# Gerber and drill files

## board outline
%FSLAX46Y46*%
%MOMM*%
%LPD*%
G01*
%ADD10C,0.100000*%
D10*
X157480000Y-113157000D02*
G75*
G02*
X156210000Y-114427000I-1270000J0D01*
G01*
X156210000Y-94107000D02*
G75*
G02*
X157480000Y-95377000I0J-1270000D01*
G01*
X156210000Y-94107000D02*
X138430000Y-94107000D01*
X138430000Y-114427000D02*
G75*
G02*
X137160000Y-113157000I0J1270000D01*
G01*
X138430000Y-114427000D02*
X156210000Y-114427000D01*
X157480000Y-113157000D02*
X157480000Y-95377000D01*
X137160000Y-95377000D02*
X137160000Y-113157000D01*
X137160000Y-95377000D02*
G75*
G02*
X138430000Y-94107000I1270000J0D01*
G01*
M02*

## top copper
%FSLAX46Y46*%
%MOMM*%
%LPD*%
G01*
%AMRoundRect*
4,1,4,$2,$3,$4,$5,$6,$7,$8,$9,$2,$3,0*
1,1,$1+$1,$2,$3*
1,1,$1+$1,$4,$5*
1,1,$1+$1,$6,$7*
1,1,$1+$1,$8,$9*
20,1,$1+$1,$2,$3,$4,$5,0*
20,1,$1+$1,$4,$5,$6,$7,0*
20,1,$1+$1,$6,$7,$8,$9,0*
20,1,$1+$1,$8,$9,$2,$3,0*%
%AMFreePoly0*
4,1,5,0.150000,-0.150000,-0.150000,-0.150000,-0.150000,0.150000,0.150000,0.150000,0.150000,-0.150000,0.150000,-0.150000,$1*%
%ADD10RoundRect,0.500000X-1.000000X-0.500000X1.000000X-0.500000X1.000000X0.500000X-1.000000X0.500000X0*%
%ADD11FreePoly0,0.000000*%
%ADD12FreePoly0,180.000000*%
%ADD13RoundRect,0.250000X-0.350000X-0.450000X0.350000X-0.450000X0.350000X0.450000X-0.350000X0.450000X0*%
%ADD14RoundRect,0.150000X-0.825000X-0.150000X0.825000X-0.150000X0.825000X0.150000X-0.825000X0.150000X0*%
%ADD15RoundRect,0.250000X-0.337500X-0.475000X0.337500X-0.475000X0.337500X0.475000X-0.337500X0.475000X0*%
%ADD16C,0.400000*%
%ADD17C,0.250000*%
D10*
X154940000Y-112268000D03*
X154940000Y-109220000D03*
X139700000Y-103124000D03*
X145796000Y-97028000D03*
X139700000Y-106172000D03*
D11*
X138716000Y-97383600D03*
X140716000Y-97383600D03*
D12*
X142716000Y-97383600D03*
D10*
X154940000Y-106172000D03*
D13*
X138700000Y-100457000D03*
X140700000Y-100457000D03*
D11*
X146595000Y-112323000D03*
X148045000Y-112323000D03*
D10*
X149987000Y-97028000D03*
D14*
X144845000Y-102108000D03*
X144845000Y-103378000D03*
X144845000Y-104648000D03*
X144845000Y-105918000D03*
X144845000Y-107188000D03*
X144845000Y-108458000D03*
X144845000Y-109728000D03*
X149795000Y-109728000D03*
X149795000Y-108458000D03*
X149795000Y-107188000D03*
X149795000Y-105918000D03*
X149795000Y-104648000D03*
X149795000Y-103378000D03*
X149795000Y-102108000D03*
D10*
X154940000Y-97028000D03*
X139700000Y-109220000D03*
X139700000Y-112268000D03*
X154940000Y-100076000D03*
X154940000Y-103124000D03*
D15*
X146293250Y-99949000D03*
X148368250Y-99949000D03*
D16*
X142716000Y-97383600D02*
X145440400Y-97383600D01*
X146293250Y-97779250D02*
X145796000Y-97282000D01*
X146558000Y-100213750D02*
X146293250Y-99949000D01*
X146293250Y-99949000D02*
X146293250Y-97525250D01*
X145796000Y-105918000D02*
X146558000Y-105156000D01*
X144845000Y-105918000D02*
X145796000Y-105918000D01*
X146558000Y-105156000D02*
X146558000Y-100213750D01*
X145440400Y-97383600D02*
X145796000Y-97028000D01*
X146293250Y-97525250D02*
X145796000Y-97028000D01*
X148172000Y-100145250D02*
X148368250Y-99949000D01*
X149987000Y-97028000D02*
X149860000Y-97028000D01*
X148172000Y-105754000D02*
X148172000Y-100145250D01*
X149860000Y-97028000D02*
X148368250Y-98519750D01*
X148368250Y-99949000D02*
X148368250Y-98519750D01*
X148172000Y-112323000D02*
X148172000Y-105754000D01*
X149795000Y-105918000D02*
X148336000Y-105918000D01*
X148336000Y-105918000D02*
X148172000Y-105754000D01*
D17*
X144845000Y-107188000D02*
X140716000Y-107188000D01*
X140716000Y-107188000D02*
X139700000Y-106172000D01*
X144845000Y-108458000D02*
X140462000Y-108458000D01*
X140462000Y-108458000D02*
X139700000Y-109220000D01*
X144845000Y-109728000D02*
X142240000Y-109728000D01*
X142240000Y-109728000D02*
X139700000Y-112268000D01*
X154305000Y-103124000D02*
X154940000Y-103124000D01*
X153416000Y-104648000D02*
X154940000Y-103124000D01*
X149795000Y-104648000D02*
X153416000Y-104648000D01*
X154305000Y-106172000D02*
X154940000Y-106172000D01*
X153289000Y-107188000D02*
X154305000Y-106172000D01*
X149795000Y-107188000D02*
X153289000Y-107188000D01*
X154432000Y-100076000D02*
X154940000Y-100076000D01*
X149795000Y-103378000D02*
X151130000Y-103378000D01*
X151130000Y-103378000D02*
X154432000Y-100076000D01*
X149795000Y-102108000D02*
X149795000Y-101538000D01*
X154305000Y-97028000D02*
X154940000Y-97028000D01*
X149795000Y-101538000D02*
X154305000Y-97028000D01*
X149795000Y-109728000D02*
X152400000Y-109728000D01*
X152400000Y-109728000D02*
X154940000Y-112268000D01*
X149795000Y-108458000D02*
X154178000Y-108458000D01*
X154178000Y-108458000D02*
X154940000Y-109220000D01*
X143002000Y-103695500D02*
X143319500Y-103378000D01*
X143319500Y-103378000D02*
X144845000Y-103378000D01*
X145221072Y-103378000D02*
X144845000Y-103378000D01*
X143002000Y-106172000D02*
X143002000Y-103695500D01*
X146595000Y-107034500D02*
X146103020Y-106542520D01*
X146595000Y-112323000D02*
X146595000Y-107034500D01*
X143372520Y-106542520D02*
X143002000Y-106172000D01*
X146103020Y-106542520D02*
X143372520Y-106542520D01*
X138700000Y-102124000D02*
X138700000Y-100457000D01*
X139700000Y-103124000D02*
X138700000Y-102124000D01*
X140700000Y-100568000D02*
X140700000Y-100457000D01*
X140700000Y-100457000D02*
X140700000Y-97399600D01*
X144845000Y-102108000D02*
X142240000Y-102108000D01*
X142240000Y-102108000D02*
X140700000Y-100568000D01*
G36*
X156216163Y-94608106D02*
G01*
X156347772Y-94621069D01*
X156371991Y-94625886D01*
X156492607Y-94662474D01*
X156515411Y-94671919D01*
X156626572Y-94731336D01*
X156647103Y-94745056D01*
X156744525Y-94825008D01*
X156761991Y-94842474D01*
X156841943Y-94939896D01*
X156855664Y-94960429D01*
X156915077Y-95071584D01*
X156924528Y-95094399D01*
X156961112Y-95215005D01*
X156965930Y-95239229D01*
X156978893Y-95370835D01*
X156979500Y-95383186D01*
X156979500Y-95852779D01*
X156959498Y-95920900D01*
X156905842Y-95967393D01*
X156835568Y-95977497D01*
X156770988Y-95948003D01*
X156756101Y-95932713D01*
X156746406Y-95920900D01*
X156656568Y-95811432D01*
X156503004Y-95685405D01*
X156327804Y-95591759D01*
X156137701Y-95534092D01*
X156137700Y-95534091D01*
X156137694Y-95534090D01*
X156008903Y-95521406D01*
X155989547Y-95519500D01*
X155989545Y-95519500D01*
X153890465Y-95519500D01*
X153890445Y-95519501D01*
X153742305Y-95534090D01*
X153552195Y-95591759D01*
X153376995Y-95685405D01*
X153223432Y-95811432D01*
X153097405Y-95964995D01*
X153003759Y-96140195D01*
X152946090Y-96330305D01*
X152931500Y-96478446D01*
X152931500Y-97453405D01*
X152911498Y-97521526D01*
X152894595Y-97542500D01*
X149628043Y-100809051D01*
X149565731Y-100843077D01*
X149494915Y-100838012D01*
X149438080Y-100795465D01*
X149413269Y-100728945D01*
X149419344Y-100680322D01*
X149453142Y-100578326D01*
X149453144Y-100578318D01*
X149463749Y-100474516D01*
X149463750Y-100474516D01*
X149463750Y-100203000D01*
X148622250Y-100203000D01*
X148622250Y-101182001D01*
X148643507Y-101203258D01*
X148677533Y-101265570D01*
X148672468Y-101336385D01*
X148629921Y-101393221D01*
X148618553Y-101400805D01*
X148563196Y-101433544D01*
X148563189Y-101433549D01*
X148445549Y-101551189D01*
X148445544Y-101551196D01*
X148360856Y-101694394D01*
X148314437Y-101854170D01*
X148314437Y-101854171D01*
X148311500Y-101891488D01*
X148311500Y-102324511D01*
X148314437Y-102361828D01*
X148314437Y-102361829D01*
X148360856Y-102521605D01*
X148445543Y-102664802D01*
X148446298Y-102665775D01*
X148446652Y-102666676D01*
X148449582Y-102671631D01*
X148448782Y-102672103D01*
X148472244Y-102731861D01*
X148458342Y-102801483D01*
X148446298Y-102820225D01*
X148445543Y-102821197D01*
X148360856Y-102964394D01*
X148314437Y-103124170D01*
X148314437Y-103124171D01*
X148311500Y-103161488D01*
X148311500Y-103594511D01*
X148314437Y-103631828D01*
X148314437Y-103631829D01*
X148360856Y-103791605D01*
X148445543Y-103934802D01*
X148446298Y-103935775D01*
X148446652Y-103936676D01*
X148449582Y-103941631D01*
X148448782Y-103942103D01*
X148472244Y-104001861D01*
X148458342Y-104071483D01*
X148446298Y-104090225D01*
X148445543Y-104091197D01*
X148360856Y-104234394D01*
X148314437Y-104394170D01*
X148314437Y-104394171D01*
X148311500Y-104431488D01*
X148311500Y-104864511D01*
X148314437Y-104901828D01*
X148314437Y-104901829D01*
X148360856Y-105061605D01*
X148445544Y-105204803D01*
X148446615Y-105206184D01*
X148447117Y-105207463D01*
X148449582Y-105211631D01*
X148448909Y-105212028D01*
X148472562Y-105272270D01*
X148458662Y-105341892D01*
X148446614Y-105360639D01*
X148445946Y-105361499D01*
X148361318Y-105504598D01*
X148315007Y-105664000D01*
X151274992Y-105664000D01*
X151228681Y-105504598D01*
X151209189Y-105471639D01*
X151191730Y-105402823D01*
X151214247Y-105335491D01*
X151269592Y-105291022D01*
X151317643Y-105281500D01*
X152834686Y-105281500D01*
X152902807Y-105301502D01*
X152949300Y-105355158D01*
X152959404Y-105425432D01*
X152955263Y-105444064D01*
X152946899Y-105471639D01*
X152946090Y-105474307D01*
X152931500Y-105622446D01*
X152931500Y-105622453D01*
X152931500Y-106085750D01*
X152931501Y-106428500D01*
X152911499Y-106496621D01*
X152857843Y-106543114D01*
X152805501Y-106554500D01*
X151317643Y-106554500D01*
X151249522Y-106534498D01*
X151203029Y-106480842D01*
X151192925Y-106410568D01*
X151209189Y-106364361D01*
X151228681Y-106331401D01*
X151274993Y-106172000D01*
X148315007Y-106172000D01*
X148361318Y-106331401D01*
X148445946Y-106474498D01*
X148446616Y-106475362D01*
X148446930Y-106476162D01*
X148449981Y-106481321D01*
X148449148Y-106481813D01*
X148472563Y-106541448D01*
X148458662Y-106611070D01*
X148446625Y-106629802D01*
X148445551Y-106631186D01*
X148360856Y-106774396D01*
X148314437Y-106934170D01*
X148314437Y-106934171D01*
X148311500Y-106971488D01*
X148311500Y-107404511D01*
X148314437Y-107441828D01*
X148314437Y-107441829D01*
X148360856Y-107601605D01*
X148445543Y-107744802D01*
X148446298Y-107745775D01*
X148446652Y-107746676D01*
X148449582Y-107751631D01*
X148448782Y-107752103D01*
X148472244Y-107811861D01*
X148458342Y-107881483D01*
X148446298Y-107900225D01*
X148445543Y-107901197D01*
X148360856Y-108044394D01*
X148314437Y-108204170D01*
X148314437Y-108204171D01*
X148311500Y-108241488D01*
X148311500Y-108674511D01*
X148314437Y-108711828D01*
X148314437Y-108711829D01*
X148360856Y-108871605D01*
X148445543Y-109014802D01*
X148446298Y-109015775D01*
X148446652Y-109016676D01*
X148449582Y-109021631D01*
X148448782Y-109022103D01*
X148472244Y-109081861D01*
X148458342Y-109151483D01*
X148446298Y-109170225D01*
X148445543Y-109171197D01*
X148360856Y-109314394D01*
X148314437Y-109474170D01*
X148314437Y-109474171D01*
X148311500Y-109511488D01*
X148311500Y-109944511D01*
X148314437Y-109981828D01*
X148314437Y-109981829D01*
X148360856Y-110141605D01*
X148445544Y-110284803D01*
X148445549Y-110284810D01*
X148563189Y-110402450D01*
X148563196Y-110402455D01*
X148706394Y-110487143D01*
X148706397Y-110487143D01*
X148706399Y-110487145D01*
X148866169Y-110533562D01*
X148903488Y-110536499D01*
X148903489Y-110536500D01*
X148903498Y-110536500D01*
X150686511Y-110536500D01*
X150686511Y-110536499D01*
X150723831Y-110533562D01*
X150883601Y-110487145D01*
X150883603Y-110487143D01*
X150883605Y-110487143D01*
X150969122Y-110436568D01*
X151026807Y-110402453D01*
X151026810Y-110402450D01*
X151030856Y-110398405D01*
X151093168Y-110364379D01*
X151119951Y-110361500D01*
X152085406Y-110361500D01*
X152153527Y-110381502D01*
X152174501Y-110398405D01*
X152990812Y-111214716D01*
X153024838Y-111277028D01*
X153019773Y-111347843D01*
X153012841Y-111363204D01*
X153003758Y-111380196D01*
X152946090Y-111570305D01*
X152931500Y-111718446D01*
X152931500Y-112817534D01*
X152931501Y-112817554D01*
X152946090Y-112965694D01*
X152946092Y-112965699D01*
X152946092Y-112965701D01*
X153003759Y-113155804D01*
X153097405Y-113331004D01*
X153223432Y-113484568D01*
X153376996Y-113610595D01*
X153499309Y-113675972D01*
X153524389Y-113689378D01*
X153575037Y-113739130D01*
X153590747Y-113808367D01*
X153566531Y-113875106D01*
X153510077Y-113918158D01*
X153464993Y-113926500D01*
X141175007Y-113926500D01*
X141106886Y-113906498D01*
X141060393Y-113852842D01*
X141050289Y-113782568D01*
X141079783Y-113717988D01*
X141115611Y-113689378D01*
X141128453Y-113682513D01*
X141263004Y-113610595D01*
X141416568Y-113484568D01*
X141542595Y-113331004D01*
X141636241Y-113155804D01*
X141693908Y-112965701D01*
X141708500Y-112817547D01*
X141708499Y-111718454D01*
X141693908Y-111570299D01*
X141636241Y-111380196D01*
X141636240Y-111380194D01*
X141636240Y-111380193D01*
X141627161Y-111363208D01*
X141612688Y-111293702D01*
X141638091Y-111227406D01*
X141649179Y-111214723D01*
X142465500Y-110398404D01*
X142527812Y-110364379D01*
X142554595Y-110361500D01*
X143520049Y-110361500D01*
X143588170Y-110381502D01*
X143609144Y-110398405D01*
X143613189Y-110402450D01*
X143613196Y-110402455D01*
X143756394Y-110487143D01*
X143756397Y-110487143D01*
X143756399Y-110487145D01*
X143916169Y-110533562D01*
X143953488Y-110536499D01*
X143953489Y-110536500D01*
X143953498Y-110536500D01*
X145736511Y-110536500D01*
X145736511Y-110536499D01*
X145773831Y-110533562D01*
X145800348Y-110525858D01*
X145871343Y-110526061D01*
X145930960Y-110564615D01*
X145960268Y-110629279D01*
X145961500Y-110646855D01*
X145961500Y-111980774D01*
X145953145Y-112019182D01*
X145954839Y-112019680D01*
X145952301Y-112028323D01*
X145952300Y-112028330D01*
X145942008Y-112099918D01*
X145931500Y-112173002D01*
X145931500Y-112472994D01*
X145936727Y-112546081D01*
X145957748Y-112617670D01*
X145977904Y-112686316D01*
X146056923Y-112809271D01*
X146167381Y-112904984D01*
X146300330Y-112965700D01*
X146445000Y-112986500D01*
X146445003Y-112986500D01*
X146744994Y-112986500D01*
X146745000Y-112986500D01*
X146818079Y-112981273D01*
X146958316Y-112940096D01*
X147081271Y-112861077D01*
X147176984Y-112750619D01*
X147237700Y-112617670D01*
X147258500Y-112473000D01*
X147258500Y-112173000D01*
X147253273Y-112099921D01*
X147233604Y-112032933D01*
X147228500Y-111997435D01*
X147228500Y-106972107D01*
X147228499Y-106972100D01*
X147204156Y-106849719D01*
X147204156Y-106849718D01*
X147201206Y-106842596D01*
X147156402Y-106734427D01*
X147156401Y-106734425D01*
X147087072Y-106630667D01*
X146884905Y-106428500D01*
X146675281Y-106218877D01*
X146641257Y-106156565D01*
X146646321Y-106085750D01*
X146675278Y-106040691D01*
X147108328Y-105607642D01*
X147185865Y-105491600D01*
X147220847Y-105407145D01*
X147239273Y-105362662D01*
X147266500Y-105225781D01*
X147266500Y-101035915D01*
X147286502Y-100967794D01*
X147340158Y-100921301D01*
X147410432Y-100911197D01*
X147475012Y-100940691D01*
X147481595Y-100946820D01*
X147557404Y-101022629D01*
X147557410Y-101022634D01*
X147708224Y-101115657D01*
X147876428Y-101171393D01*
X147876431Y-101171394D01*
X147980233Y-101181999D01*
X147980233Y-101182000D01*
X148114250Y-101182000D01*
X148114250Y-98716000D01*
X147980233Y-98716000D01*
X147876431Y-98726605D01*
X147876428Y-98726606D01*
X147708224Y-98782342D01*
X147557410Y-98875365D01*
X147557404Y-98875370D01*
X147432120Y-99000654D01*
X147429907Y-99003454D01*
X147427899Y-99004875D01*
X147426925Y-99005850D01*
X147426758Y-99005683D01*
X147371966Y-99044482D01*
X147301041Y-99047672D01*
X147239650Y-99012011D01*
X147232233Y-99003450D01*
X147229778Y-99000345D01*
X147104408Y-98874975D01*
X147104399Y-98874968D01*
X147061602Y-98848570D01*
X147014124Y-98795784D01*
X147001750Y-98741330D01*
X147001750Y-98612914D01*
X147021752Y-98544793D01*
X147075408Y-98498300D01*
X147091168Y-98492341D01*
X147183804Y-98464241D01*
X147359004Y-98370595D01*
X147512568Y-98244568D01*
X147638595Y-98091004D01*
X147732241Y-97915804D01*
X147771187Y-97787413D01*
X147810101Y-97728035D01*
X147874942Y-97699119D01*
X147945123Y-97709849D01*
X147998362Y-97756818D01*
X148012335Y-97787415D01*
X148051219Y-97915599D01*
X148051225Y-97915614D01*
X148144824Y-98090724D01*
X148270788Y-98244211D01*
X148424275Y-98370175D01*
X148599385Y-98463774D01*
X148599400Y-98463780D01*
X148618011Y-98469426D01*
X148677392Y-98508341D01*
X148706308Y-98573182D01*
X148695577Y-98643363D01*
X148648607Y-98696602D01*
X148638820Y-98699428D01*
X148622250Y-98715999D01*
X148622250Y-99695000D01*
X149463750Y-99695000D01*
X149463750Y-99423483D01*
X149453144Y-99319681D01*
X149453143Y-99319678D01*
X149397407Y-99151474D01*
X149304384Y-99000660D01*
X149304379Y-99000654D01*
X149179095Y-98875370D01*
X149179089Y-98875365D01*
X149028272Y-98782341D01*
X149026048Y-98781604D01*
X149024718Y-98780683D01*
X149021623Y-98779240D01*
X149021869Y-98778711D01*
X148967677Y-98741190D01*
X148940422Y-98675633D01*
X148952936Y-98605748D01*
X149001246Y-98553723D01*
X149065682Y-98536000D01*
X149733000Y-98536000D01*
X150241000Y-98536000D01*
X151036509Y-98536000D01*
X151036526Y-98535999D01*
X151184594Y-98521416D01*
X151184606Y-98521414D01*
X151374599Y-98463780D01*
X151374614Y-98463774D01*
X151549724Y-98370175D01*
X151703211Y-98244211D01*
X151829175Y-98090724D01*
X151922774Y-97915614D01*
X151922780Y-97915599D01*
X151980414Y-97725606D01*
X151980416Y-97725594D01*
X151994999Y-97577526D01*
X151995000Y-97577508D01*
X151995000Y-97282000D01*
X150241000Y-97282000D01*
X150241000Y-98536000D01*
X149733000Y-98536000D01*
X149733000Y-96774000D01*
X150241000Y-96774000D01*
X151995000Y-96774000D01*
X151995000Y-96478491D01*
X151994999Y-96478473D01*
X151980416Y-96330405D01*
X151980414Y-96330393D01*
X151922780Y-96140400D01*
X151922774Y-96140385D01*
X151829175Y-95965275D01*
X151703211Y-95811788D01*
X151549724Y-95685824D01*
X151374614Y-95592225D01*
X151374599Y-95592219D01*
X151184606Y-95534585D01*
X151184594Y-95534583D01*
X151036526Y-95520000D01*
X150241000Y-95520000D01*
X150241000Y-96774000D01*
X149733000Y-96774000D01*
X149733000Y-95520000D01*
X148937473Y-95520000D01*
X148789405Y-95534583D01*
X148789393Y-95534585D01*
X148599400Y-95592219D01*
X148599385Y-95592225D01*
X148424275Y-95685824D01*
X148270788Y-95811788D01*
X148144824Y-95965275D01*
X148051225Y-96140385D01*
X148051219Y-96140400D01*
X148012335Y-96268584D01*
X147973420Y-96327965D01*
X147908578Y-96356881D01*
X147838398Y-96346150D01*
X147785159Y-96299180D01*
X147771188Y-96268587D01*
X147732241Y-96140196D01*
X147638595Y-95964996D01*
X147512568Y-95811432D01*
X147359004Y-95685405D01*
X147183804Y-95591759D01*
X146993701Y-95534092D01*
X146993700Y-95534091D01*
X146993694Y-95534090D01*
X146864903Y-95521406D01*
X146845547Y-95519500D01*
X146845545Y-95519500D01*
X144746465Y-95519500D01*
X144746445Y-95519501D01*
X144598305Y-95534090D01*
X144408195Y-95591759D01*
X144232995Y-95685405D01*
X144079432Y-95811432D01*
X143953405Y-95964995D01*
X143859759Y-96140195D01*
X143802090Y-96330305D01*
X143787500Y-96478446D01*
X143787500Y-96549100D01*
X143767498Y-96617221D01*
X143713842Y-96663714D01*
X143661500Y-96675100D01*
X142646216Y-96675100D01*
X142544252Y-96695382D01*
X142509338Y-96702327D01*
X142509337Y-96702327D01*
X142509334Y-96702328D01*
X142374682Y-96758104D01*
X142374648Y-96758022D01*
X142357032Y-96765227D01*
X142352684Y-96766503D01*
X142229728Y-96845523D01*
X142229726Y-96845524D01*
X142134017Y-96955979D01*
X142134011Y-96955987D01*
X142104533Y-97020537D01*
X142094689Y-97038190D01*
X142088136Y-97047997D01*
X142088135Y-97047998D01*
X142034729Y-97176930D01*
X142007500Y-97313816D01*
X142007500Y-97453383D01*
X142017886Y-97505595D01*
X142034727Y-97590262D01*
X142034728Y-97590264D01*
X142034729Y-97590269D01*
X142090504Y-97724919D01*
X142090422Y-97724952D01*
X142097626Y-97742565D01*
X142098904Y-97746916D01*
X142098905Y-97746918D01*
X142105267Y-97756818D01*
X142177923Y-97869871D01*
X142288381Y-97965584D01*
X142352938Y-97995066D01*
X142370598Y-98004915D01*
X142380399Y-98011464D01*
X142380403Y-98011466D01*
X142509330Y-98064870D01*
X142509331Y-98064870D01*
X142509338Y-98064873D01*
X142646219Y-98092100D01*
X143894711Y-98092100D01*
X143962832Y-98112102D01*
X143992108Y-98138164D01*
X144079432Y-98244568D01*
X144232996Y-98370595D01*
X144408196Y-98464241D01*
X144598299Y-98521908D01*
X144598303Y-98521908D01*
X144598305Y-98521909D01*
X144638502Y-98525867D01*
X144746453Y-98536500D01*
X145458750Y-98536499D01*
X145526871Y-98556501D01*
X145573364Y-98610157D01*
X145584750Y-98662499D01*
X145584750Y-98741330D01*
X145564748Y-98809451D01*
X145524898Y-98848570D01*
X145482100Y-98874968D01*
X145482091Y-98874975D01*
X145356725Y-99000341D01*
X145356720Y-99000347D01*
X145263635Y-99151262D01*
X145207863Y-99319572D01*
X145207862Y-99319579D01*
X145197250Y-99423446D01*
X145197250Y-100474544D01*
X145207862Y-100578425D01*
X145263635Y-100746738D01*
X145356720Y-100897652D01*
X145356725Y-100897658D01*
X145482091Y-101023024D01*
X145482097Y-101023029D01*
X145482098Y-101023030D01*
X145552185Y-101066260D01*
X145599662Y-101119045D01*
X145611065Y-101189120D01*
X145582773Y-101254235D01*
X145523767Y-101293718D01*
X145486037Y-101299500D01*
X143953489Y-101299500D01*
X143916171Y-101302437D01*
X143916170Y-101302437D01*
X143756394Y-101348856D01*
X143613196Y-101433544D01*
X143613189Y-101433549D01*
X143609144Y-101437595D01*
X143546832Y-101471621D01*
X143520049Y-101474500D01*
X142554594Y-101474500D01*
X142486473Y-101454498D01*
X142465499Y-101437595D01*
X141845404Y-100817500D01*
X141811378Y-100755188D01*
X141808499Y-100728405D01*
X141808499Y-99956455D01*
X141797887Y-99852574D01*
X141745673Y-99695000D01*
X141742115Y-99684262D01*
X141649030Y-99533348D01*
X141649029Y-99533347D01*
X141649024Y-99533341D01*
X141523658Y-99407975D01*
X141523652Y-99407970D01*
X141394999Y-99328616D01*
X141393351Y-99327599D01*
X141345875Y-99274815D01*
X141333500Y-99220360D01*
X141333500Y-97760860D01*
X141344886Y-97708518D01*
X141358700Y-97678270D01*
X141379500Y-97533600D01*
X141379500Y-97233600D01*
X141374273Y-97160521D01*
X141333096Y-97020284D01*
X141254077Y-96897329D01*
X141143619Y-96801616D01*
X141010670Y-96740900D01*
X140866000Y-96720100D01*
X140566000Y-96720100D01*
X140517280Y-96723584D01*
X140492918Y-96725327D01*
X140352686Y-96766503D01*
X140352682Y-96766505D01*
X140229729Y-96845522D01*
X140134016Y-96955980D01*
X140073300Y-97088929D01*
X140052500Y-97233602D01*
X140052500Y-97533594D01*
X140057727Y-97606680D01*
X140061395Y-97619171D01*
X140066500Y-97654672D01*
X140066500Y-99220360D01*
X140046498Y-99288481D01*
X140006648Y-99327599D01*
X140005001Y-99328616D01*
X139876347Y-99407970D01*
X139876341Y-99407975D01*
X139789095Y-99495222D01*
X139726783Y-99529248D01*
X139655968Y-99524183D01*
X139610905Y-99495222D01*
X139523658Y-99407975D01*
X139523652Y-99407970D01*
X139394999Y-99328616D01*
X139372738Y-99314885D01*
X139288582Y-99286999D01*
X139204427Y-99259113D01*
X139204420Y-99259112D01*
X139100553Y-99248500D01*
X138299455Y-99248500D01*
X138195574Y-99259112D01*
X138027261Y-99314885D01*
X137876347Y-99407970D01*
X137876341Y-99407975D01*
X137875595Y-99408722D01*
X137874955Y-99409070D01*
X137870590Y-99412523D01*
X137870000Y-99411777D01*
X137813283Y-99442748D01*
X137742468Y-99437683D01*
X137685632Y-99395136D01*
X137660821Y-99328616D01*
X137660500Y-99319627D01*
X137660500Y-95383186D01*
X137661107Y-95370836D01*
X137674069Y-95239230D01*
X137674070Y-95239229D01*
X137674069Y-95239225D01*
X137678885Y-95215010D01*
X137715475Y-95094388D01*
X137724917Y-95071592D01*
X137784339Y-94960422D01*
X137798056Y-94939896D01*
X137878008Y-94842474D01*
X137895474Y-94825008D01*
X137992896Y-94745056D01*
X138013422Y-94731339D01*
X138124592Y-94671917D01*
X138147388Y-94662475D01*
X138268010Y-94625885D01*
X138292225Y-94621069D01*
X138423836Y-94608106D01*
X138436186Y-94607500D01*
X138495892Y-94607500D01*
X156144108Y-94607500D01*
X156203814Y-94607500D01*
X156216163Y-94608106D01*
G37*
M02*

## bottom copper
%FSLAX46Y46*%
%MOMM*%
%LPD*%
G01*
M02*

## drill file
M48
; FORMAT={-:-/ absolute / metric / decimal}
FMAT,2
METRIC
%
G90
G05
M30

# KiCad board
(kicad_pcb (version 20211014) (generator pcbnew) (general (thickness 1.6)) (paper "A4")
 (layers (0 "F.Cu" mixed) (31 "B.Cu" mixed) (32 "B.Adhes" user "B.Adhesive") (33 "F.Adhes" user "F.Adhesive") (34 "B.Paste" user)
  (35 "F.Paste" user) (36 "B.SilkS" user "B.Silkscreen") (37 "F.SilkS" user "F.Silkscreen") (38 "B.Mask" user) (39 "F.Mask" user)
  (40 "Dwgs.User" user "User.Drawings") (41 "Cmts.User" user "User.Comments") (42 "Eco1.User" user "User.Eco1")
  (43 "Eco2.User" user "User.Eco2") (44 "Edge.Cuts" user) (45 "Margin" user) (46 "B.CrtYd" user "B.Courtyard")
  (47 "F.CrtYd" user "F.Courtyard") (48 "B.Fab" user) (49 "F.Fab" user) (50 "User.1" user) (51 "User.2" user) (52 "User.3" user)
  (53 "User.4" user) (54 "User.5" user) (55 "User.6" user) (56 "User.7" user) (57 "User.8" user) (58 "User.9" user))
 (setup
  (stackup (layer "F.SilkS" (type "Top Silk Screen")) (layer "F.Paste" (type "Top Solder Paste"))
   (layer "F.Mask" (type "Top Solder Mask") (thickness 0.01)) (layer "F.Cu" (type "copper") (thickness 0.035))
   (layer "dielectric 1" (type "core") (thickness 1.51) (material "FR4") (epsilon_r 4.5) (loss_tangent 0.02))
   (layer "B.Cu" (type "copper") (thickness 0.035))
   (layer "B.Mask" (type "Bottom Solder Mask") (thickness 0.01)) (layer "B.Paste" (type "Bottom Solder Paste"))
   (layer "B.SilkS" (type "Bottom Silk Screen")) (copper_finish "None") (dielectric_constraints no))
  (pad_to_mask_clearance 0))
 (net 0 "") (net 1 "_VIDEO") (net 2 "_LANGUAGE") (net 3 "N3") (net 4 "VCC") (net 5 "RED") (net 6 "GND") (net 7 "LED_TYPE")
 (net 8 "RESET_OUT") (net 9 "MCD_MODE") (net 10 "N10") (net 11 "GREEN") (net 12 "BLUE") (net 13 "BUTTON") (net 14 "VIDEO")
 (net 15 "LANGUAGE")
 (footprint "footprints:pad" (layer "F.Cu") (at 154.94 112.268)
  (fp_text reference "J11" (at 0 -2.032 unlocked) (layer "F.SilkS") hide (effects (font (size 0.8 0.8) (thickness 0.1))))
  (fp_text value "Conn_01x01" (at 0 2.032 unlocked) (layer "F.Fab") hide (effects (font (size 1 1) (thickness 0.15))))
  (pad "1" smd roundrect (at 0 0) (size 3 2) (layers "F.Cu" "F.Paste" "F.Mask") (roundrect_rratio 0.25) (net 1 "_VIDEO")))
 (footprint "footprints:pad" (layer "F.Cu") (at 154.94 109.22)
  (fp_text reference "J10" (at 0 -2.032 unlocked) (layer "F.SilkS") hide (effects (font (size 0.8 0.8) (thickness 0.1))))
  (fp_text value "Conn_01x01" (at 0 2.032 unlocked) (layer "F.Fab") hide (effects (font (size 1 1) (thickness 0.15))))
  (pad "1" smd roundrect (at 0 0) (size 3 2) (layers "F.Cu" "F.Paste" "F.Mask") (roundrect_rratio 0.25) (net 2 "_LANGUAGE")))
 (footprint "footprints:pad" (layer "F.Cu") (at 139.7 103.124)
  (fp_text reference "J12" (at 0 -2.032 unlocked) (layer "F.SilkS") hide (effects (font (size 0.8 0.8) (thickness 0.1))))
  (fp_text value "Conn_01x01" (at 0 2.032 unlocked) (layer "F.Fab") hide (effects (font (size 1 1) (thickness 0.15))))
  (pad "1" smd roundrect (at 0 0) (size 3 2) (layers "F.Cu" "F.Paste" "F.Mask") (roundrect_rratio 0.25) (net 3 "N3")))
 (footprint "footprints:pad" (layer "F.Cu") (at 145.796 97.028)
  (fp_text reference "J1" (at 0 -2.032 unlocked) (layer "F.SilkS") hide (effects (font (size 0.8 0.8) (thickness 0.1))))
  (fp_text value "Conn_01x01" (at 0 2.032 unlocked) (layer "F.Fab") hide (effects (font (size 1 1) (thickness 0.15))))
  (pad "1" smd roundrect (at 0 0) (size 3 2) (layers "F.Cu" "F.Paste" "F.Mask") (roundrect_rratio 0.25) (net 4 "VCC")))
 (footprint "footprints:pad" (layer "F.Cu") (at 139.7 106.172)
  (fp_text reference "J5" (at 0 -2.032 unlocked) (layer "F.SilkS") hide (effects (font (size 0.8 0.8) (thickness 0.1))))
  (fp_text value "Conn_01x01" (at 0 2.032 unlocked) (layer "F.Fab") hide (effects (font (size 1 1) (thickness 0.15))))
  (pad "1" smd roundrect (at 0 0) (size 3 2) (layers "F.Cu" "F.Paste" "F.Mask") (roundrect_rratio 0.25) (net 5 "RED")))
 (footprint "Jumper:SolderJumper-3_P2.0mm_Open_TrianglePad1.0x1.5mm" (layer "F.Cu") (at 140.716 97.3836)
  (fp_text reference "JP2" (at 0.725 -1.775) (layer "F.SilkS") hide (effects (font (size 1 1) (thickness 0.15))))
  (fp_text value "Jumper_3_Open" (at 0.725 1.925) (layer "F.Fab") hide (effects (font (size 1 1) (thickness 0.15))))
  (pad "" smd rect (at -1.2 0) (size 1.5 1.5) (layers "F.Mask"))
  (pad "" smd rect (at 1.2 0) (size 1.5 1.5) (layers "F.Mask"))
  (pad "1" smd custom (at -2 0) (size 0.3 0.3) (layers "F.Cu" "F.Mask") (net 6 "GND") (zone_connect 2)
   (options (clearance outline) (anchor rect)) (primitives))
  (pad "2" smd custom (at 0 0) (size 0.3 0.3) (layers "F.Cu") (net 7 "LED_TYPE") (zone_connect 2)
   (options (clearance outline) (anchor rect)) (primitives))
  (pad "3" smd custom (at 2 0 180) (size 0.3 0.3) (layers "F.Cu" "F.Mask") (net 4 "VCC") (zone_connect 2)
   (options (clearance outline) (anchor rect)) (primitives)))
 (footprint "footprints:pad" (layer "F.Cu") (at 154.94 106.172)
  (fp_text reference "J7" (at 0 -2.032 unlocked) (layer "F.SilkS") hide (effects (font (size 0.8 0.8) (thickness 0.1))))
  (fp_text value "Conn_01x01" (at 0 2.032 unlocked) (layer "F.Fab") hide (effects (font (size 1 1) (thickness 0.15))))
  (pad "1" smd roundrect (at 0 0) (size 3 2) (layers "F.Cu" "F.Paste" "F.Mask") (roundrect_rratio 0.25) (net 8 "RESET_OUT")))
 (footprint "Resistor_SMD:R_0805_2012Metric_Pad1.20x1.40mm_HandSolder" (layer "F.Cu") (at 139.7 100.457)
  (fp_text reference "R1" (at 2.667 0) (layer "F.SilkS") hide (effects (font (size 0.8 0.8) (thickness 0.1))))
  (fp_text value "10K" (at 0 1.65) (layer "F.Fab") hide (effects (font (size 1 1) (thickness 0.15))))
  (pad "1" smd roundrect (at -1 0) (size 1.2 1.4) (layers "F.Cu" "F.Paste" "F.Mask") (roundrect_rratio 0.2083333333) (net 3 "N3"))
  (pad "2" smd roundrect (at 1 0) (size 1.2 1.4) (layers "F.Cu" "F.Paste" "F.Mask") (roundrect_rratio 0.2083333333) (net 7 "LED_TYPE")))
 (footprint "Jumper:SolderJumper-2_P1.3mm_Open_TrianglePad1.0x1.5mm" (layer "F.Cu") (at 147.32 112.323)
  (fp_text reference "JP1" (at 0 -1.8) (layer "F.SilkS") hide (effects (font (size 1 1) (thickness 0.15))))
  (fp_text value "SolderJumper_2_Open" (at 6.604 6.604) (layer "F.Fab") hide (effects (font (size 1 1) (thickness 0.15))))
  (pad "1" smd custom (at -0.725 0) (size 0.3 0.3) (layers "F.Cu" "F.Mask") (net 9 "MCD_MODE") (zone_connect 2)
   (options (clearance outline) (anchor rect)) (primitives))
  (pad "2" smd custom (at 0.725 0) (size 0.3 0.3) (layers "F.Cu" "F.Mask") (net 6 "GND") (zone_connect 2)
   (options (clearance outline) (anchor rect)) (primitives)))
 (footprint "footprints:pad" (layer "F.Cu") (at 149.987 97.028)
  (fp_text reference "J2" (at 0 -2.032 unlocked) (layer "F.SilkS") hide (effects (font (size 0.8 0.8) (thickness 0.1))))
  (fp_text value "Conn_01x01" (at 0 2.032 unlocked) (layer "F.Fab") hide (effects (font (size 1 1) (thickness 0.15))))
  (pad "1" smd roundrect (at 0 0) (size 3 2) (layers "F.Cu" "F.Paste" "F.Mask") (roundrect_rratio 0.25) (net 6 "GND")))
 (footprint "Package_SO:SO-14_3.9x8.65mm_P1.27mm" (layer "F.Cu") (at 147.32 105.918)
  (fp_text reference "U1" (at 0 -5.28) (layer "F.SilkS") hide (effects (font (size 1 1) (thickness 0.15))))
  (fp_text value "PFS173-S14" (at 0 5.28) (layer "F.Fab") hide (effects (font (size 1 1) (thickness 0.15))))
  (pad "1" smd roundrect (at -2.475 -3.81) (size 1.95 0.6) (layers "F.Cu" "F.Paste" "F.Mask") (roundrect_rratio 0.25) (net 7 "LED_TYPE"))
  (pad "2" smd roundrect (at -2.475 -2.54) (size 1.95 0.6) (layers "F.Cu" "F.Paste" "F.Mask") (roundrect_rratio 0.25) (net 9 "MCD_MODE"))
  (pad "3" smd roundrect (at -2.475 -1.27) (size 1.95 0.6) (layers "F.Cu" "F.Paste" "F.Mask") (roundrect_rratio 0.25) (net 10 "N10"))
  (pad "4" smd roundrect (at -2.475 0) (size 1.95 0.6) (layers "F.Cu" "F.Paste" "F.Mask") (roundrect_rratio 0.25) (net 4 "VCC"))
  (pad "5" smd roundrect (at -2.475 1.27) (size 1.95 0.6) (layers "F.Cu" "F.Paste" "F.Mask") (roundrect_rratio 0.25) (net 5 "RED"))
  (pad "6" smd roundrect (at -2.475 2.54) (size 1.95 0.6) (layers "F.Cu" "F.Paste" "F.Mask") (roundrect_rratio 0.25) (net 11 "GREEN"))
  (pad "7" smd roundrect (at -2.475 3.81) (size 1.95 0.6) (layers "F.Cu" "F.Paste" "F.Mask") (roundrect_rratio 0.25) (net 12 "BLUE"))
  (pad "8" smd roundrect (at 2.475 3.81) (size 1.95 0.6) (layers "F.Cu" "F.Paste" "F.Mask") (roundrect_rratio 0.25) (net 1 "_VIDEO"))
  (pad "9" smd roundrect (at 2.475 2.54) (size 1.95 0.6) (layers "F.Cu" "F.Paste" "F.Mask") (roundrect_rratio 0.25) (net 2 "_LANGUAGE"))
  (pad "10" smd roundrect (at 2.475 1.27) (size 1.95 0.6) (layers "F.Cu" "F.Paste" "F.Mask") (roundrect_rratio 0.25) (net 8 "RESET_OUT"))
  (pad "11" smd roundrect (at 2.475 0) (size 1.95 0.6) (layers "F.Cu" "F.Paste" "F.Mask") (roundrect_rratio 0.25) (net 6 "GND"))
  (pad "12" smd roundrect (at 2.475 -1.27) (size 1.95 0.6) (layers "F.Cu" "F.Paste" "F.Mask") (roundrect_rratio 0.25) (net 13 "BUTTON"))
  (pad "13" smd roundrect (at 2.475 -2.54) (size 1.95 0.6) (layers "F.Cu" "F.Paste" "F.Mask") (roundrect_rratio 0.25) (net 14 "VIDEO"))
  (pad "14" smd roundrect (at 2.475 -3.81) (size 1.95 0.6) (layers "F.Cu" "F.Paste" "F.Mask") (roundrect_rratio 0.25) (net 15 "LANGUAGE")))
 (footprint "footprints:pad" (layer "F.Cu") (at 154.94 97.028)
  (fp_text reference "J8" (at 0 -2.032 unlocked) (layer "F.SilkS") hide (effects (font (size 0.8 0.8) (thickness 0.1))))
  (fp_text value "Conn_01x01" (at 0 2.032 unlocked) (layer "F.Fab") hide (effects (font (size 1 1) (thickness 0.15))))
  (pad "1" smd roundrect (at 0 0) (size 3 2) (layers "F.Cu" "F.Paste" "F.Mask") (roundrect_rratio 0.25) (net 15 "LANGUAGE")))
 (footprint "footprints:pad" (layer "F.Cu") (at 139.7 109.22)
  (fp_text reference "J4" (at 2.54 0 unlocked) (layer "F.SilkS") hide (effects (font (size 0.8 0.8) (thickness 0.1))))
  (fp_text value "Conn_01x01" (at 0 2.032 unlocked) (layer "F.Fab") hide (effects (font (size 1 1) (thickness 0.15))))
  (pad "1" smd roundrect (at 0 0) (size 3 2) (layers "F.Cu" "F.Paste" "F.Mask") (roundrect_rratio 0.25) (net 11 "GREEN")))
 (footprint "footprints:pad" (layer "F.Cu") (at 139.7 112.268)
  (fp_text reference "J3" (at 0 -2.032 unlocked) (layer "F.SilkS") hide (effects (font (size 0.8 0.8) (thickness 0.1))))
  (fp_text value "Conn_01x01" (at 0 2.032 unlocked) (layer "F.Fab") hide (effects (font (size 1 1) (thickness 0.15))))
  (pad "1" smd roundrect (at 0 0) (size 3 2) (layers "F.Cu" "F.Paste" "F.Mask") (roundrect_rratio 0.25) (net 12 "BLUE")))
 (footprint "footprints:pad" (layer "F.Cu") (at 154.94 100.076)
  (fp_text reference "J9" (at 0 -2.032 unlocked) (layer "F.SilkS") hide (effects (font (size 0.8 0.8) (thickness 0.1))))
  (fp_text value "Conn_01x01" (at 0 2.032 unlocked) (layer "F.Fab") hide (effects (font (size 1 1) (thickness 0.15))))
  (pad "1" smd roundrect (at 0 0) (size 3 2) (layers "F.Cu" "F.Paste" "F.Mask") (roundrect_rratio 0.25) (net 14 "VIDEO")))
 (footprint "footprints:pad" (layer "F.Cu") (at 154.94 103.124)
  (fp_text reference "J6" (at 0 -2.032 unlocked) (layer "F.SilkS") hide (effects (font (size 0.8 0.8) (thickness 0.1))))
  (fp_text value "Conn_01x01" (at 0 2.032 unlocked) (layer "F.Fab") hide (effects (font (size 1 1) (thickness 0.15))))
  (pad "1" smd roundrect (at 0 0) (size 3 2) (layers "F.Cu" "F.Paste" "F.Mask") (roundrect_rratio 0.25) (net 13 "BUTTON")))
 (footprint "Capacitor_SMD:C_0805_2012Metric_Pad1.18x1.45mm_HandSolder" (layer "F.Cu") (at 147.33075 99.949)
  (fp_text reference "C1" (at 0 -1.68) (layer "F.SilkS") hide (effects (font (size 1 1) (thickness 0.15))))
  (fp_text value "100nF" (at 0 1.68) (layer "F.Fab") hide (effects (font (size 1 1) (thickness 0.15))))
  (pad "1" smd roundrect (at -1.0375 0) (size 1.175 1.45) (layers "F.Cu" "F.Paste" "F.Mask") (roundrect_rratio 0.2127659574) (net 4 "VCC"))
  (pad "2" smd roundrect (at 1.0375 0) (size 1.175 1.45) (layers "F.Cu" "F.Paste" "F.Mask") (roundrect_rratio 0.2127659574) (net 6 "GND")))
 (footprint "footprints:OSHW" (layer "B.Cu") (at 144.399 98.298 180)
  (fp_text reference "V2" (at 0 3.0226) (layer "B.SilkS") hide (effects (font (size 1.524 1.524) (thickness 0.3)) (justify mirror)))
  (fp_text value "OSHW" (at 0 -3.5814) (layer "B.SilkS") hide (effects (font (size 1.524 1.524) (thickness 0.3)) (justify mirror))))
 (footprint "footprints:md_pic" (layer "B.Cu") (at 151.257 98.171 180)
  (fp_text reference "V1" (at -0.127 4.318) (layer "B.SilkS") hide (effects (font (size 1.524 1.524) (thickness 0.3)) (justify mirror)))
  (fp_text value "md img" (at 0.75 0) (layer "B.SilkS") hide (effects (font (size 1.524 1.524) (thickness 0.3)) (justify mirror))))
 (gr_arc (start 157.48 113.157) (mid 157.108026 114.055026) (end 156.21 114.427) (layer "Edge.Cuts") (width 0.1))
 (gr_arc (start 156.21 94.107) (mid 157.108026 94.478974) (end 157.48 95.377) (layer "Edge.Cuts") (width 0.1))
 (gr_line (start 156.21 94.107) (end 138.43 94.107) (layer "Edge.Cuts") (width 0.1))
 (gr_arc (start 138.43 114.427) (mid 137.531974 114.055026) (end 137.16 113.157) (layer "Edge.Cuts") (width 0.1))
 (gr_line (start 138.43 114.427) (end 156.21 114.427) (layer "Edge.Cuts") (width 0.1))
 (gr_line (start 157.48 113.157) (end 157.48 95.377) (layer "Edge.Cuts") (width 0.1))
 (gr_line (start 137.16 95.377) (end 137.16 113.157) (layer "Edge.Cuts") (width 0.1))
 (gr_arc (start 137.16 95.377) (mid 137.531974 94.478974) (end 138.43 94.107) (layer "Edge.Cuts") (width 0.1))
 (segment (start 142.716 97.3836) (end 145.4404 97.3836) (width 0.4) (layer "F.Cu") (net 4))
 (segment (start 146.29325 97.77925) (end 145.796 97.282) (width 0.4) (layer "F.Cu") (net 4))
 (segment (start 146.558 100.21375) (end 146.29325 99.949) (width 0.4) (layer "F.Cu") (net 4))
 (segment (start 146.29325 99.949) (end 146.29325 97.52525) (width 0.4) (layer "F.Cu") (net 4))
 (segment (start 145.796 105.918) (end 146.558 105.156) (width 0.4) (layer "F.Cu") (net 4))
 (segment (start 144.845 105.918) (end 145.796 105.918) (width 0.4) (layer "F.Cu") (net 4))
 (segment (start 146.558 105.156) (end 146.558 100.21375) (width 0.4) (layer "F.Cu") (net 4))
 (segment (start 145.4404 97.3836) (end 145.796 97.028) (width 0.4) (layer "F.Cu") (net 4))
 (segment (start 146.29325 97.52525) (end 145.796 97.028) (width 0.4) (layer "F.Cu") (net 4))
 (segment (start 148.172 100.14525) (end 148.36825 99.949) (width 0.4) (layer "F.Cu") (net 6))
 (segment (start 149.987 97.028) (end 149.86 97.028) (width 0.4) (layer "F.Cu") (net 6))
 (segment (start 148.172 105.754) (end 148.172 100.14525) (width 0.4) (layer "F.Cu") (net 6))
 (segment (start 149.86 97.028) (end 148.36825 98.51975) (width 0.4) (layer "F.Cu") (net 6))
 (segment (start 148.36825 99.949) (end 148.36825 98.51975) (width 0.4) (layer "F.Cu") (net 6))
 (segment (start 148.172 112.323) (end 148.172 105.754) (width 0.4) (layer "F.Cu") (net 6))
 (segment (start 149.795 105.918) (end 148.336 105.918) (width 0.4) (layer "F.Cu") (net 6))
 (segment (start 148.336 105.918) (end 148.172 105.754) (width 0.4) (layer "F.Cu") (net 6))
 (segment (start 144.845 107.188) (end 140.716 107.188) (width 0.25) (layer "F.Cu") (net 5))
 (segment (start 140.716 107.188) (end 139.7 106.172) (width 0.25) (layer "F.Cu") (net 5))
 (segment (start 144.845 108.458) (end 140.462 108.458) (width 0.25) (layer "F.Cu") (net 11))
 (segment (start 140.462 108.458) (end 139.7 109.22) (width 0.25) (layer "F.Cu") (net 11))
 (segment (start 144.845 109.728) (end 142.24 109.728) (width 0.25) (layer "F.Cu") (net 12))
 (segment (start 142.24 109.728) (end 139.7 112.268) (width 0.25) (layer "F.Cu") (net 12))
 (segment (start 154.305 103.124) (end 154.94 103.124) (width 0.25) (layer "F.Cu") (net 13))
 (segment (start 153.416 104.648) (end 154.94 103.124) (width 0.25) (layer "F.Cu") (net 13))
 (segment (start 149.795 104.648) (end 153.416 104.648) (width 0.25) (layer "F.Cu") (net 13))
 (segment (start 154.305 106.172) (end 154.94 106.172) (width 0.25) (layer "F.Cu") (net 8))
 (segment (start 153.289 107.188) (end 154.305 106.172) (width 0.25) (layer "F.Cu") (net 8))
 (segment (start 149.795 107.188) (end 153.289 107.188) (width 0.25) (layer "F.Cu") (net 8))
 (segment (start 154.432 100.076) (end 154.94 100.076) (width 0.25) (layer "F.Cu") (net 14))
 (segment (start 149.795 103.378) (end 151.13 103.378) (width 0.25) (layer "F.Cu") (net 14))
 (segment (start 151.13 103.378) (end 154.432 100.076) (width 0.25) (layer "F.Cu") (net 14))
 (segment (start 149.795 102.108) (end 149.795 101.538) (width 0.25) (layer "F.Cu") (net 15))
 (segment (start 154.305 97.028) (end 154.94 97.028) (width 0.25) (layer "F.Cu") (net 15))
 (segment (start 149.795 101.538) (end 154.305 97.028) (width 0.25) (layer "F.Cu") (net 15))
 (segment (start 149.795 109.728) (end 152.4 109.728) (width 0.25) (layer "F.Cu") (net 1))
 (segment (start 152.4 109.728) (end 154.94 112.268) (width 0.25) (layer "F.Cu") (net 1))
 (segment (start 149.795 108.458) (end 154.178 108.458) (width 0.25) (layer "F.Cu") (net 2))
 (segment (start 154.178 108.458) (end 154.94 109.22) (width 0.25) (layer "F.Cu") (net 2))
 (segment (start 143.002 103.6955) (end 143.3195 103.378) (width 0.25) (layer "F.Cu") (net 9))
 (segment (start 143.3195 103.378) (end 144.845 103.378) (width 0.25) (layer "F.Cu") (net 9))
 (segment (start 145.221072 103.378) (end 144.845 103.378) (width 0.25) (layer "F.Cu") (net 9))
 (segment (start 143.002 106.172) (end 143.002 103.6955) (width 0.25) (layer "F.Cu") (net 9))
 (segment (start 146.595 107.0345) (end 146.10302 106.54252) (width 0.25) (layer "F.Cu") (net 9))
 (segment (start 146.595 112.323) (end 146.595 107.0345) (width 0.25) (layer "F.Cu") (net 9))
 (segment (start 143.37252 106.54252) (end 143.002 106.172) (width 0.25) (layer "F.Cu") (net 9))
 (segment (start 146.10302 106.54252) (end 143.37252 106.54252) (width 0.25) (layer "F.Cu") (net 9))
 (segment (start 138.7 102.124) (end 138.7 100.457) (width 0.25) (layer "F.Cu") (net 3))
 (segment (start 139.7 103.124) (end 138.7 102.124) (width 0.25) (layer "F.Cu") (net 3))
 (segment (start 140.7 100.568) (end 140.7 100.457) (width 0.25) (layer "F.Cu") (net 7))
 (segment (start 140.7 100.457) (end 140.7 97.3996) (width 0.25) (layer "F.Cu") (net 7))
 (segment (start 144.845 102.108) (end 142.24 102.108) (width 0.25) (layer "F.Cu") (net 7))
 (segment (start 142.24 102.108) (end 140.7 100.568) (width 0.25) (layer "F.Cu") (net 7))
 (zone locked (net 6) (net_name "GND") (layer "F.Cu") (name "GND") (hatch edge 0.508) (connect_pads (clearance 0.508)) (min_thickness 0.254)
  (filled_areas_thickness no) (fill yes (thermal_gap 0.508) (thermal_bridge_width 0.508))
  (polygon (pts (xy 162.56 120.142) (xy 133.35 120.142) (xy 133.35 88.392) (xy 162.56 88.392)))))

